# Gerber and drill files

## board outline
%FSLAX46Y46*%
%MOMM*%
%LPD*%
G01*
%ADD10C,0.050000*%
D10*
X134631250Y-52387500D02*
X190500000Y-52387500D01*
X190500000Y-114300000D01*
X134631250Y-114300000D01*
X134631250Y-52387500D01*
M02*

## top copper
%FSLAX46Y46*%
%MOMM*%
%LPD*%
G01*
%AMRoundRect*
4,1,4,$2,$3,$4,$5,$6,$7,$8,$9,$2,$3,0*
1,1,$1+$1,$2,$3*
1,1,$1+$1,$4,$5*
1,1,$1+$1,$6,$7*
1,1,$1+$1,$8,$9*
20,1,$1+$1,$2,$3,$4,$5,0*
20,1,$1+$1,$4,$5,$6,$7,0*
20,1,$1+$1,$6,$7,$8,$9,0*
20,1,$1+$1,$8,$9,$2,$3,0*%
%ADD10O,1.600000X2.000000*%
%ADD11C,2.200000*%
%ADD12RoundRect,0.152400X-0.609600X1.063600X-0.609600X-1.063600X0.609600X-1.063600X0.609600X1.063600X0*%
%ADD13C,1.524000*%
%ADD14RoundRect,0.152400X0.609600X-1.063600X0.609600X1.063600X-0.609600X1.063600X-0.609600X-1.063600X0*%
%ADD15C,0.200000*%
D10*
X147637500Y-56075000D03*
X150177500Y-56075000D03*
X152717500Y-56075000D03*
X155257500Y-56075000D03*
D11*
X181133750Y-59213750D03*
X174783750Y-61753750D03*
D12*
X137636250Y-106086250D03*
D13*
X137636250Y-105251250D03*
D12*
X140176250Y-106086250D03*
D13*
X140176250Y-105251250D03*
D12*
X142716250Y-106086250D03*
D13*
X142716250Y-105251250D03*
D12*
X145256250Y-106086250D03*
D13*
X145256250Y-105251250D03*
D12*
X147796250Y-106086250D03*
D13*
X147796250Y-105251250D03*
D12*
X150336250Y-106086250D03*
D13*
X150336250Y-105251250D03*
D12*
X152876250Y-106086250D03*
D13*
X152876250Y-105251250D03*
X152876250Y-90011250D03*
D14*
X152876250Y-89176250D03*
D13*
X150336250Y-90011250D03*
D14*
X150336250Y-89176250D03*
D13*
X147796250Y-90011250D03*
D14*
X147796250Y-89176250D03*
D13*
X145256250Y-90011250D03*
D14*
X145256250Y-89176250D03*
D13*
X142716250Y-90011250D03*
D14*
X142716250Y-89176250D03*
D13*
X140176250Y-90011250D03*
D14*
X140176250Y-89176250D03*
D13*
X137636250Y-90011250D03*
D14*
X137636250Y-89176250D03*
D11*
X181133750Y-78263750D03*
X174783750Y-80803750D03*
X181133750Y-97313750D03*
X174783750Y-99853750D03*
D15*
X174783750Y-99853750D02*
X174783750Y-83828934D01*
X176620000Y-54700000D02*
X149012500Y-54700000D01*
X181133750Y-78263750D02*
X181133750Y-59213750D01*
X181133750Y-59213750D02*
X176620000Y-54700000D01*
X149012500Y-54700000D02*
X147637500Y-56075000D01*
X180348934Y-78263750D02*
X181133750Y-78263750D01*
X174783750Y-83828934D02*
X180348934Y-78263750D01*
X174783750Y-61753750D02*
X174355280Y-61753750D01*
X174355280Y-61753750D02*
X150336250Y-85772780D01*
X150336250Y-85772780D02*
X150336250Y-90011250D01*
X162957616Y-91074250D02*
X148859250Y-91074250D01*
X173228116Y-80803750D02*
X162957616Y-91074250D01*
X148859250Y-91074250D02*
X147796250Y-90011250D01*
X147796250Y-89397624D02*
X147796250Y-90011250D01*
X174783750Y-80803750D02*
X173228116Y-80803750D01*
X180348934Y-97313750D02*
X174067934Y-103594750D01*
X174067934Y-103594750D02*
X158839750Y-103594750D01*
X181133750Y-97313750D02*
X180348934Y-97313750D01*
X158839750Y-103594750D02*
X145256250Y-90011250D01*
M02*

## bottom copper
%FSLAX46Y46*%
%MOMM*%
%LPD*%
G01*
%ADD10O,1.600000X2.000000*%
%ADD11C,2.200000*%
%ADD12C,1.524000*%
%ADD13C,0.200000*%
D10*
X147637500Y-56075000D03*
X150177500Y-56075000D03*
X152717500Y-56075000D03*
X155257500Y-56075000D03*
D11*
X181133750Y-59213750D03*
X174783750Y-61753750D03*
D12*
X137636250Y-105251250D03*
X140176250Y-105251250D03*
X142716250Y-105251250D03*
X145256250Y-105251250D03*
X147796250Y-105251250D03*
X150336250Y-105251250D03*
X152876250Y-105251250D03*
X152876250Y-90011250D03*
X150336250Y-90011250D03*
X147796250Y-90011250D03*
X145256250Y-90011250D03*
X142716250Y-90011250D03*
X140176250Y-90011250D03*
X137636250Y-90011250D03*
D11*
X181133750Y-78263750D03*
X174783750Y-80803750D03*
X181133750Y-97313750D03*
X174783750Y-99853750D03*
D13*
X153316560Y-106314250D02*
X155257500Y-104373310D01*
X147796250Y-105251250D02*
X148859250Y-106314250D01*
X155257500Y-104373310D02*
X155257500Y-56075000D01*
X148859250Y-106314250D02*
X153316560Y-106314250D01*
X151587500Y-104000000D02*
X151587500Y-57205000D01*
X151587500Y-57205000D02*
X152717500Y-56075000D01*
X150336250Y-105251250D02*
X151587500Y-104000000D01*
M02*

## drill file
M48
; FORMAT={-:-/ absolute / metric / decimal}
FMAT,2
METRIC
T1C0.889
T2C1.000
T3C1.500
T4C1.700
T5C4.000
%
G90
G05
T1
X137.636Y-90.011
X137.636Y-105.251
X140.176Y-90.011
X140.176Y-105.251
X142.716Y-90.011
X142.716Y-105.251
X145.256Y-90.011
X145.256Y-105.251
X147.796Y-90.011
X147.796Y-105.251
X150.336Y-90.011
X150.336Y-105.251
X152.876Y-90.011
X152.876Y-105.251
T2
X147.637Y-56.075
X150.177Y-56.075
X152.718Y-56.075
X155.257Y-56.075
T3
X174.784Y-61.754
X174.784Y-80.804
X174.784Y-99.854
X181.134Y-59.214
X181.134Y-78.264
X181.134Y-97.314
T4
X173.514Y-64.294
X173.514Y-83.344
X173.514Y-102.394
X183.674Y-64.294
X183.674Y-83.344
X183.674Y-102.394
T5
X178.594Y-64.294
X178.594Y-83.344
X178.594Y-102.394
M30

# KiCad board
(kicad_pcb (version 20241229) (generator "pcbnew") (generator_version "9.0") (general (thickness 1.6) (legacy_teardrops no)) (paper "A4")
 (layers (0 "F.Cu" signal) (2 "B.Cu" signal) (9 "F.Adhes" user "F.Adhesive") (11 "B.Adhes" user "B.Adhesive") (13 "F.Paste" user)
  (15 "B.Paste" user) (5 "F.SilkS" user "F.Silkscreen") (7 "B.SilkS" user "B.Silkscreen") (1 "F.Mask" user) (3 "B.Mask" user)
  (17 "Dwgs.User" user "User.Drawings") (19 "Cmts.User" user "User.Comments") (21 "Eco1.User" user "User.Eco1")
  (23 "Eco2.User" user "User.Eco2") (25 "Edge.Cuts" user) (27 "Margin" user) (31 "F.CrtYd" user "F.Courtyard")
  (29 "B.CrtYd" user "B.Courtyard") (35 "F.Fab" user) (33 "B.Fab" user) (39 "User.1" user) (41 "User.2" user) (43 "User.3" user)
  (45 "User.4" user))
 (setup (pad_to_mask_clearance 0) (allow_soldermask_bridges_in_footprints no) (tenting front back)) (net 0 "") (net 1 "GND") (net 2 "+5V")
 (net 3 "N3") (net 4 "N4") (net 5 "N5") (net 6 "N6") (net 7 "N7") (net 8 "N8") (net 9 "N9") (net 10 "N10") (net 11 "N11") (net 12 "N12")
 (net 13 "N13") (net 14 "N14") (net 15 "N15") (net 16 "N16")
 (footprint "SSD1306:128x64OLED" (layer "F.Cu") (at 151.2575 66.675)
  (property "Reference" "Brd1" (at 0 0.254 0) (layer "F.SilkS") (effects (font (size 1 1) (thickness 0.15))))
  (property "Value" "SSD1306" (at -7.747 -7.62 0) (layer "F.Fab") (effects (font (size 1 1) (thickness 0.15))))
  (pad "1" thru_hole oval (at -3.62 -10.6 90) (size 2 1.6) (drill 1) (layers "*.Cu" "*.Mask") (remove_unused_layers no) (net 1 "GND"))
  (pad "2" thru_hole oval (at -1.08 -10.6 90) (size 2 1.6) (drill 1) (layers "*.Cu" "*.Mask") (remove_unused_layers no) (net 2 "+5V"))
  (pad "3" thru_hole oval (at 1.46 -10.6 90) (size 2 1.6) (drill 1) (layers "*.Cu" "*.Mask") (remove_unused_layers no) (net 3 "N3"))
  (pad "4" thru_hole oval (at 4 -10.6 90) (size 2 1.6) (drill 1) (layers "*.Cu" "*.Mask") (remove_unused_layers no) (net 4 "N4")))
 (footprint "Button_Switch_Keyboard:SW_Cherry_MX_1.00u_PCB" (layer "F.Cu") (at 181.13375 59.21375)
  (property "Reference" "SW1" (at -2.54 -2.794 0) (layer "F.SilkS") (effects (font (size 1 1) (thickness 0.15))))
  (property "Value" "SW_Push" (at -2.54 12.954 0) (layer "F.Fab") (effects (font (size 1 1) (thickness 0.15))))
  (pad "" np_thru_hole circle (at -7.62 5.08) (size 1.7 1.7) (drill 1.7) (layers "*.Cu" "*.Mask"))
  (pad "" np_thru_hole circle (at -2.54 5.08) (size 4 4) (drill 4) (layers "*.Cu" "*.Mask"))
  (pad "" np_thru_hole circle (at 2.54 5.08) (size 1.7 1.7) (drill 1.7) (layers "*.Cu" "*.Mask"))
  (pad "1" thru_hole circle (at 0 0) (size 2.2 2.2) (drill 1.5) (layers "*.Cu" "*.Mask") (remove_unused_layers no) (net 1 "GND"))
  (pad "2" thru_hole circle (at -6.35 2.54) (size 2.2 2.2) (drill 1.5) (layers "*.Cu" "*.Mask") (remove_unused_layers no) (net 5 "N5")))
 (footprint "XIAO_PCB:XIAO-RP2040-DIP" (layer "F.Cu") (at 145.25625 97.63125 90)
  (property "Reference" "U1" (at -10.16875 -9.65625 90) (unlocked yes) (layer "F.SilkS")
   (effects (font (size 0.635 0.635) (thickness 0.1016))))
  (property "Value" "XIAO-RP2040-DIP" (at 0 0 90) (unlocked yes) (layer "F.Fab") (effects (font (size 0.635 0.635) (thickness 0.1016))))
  (pad "1" smd roundrect (at -8.455 -7.62 270) (size 2.432 1.524) (layers "F.Cu" "F.Mask") (roundrect_rratio 0.1) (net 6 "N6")
   (thermal_bridge_angle 45))
  (pad "1" thru_hole circle (at -7.62 -7.62 270) (size 1.524 1.524) (drill 0.889) (layers "*.Cu" "*.Mask") (remove_unused_layers no)
   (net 6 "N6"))
  (pad "2" smd roundrect (at -8.455 -5.08 270) (size 2.432 1.524) (layers "F.Cu" "F.Mask") (roundrect_rratio 0.1) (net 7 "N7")
   (thermal_bridge_angle 45))
  (pad "2" thru_hole circle (at -7.62 -5.08 270) (size 1.524 1.524) (drill 0.889) (layers "*.Cu" "*.Mask") (remove_unused_layers no)
   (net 7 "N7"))
  (pad "3" smd roundrect (at -8.455 -2.54 270) (size 2.432 1.524) (layers "F.Cu" "F.Mask") (roundrect_rratio 0.1) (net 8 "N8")
   (thermal_bridge_angle 45))
  (pad "3" thru_hole circle (at -7.62 -2.54 270) (size 1.524 1.524) (drill 0.889) (layers "*.Cu" "*.Mask") (remove_unused_layers no)
   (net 8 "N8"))
  (pad "4" smd roundrect (at -8.455 0 270) (size 2.432 1.524) (layers "F.Cu" "F.Mask") (roundrect_rratio 0.1) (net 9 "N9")
   (thermal_bridge_angle 45))
  (pad "4" thru_hole circle (at -7.62 0 270) (size 1.524 1.524) (drill 0.889) (layers "*.Cu" "*.Mask") (remove_unused_layers no)
   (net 9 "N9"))
  (pad "5" smd roundrect (at -8.455 2.54 270) (size 2.432 1.524) (layers "F.Cu" "F.Mask") (roundrect_rratio 0.1) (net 4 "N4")
   (thermal_bridge_angle 45))
  (pad "5" thru_hole circle (at -7.62 2.54 270) (size 1.524 1.524) (drill 0.889) (layers "*.Cu" "*.Mask") (remove_unused_layers no)
   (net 4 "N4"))
  (pad "6" smd roundrect (at -8.455 5.08 270) (size 2.432 1.524) (layers "F.Cu" "F.Mask") (roundrect_rratio 0.1) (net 3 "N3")
   (thermal_bridge_angle 45))
  (pad "6" thru_hole circle (at -7.62 5.08 270) (size 1.524 1.524) (drill 0.889) (layers "*.Cu" "*.Mask") (remove_unused_layers no)
   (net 3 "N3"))
  (pad "7" smd roundrect (at -8.455 7.62 270) (size 2.432 1.524) (layers "F.Cu" "F.Mask") (roundrect_rratio 0.1) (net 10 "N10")
   (thermal_bridge_angle 45))
  (pad "7" thru_hole circle (at -7.62 7.62 270) (size 1.524 1.524) (drill 0.889) (layers "*.Cu" "*.Mask") (remove_unused_layers no)
   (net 10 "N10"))
  (pad "8" thru_hole circle (at 7.62 7.62 90) (size 1.524 1.524) (drill 0.889) (layers "*.Cu" "*.Mask") (remove_unused_layers no)
   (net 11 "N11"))
  (pad "8" smd roundrect (at 8.455 7.62 90) (size 2.432 1.524) (layers "F.Cu" "F.Mask") (roundrect_rratio 0.1) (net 11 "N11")
   (thermal_bridge_angle 45))
  (pad "9" thru_hole circle (at 7.62 5.08 90) (size 1.524 1.524) (drill 0.889) (layers "*.Cu" "*.Mask") (remove_unused_layers no)
   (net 5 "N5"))
  (pad "9" smd roundrect (at 8.455 5.08 90) (size 2.432 1.524) (layers "F.Cu" "F.Mask") (roundrect_rratio 0.1) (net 5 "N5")
   (thermal_bridge_angle 45))
  (pad "10" thru_hole circle (at 7.62 2.54 90) (size 1.524 1.524) (drill 0.889) (layers "*.Cu" "*.Mask") (remove_unused_layers no)
   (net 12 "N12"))
  (pad "10" smd roundrect (at 8.455 2.54 90) (size 2.432 1.524) (layers "F.Cu" "F.Mask") (roundrect_rratio 0.1) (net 12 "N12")
   (thermal_bridge_angle 45))
  (pad "11" thru_hole circle (at 7.62 0 90) (size 1.524 1.524) (drill 0.889) (layers "*.Cu" "*.Mask") (remove_unused_layers no)
   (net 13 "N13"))
  (pad "11" smd roundrect (at 8.455 0 90) (size 2.432 1.524) (layers "F.Cu" "F.Mask") (roundrect_rratio 0.1) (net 13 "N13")
   (thermal_bridge_angle 45))
  (pad "12" thru_hole circle (at 7.62 -2.54 90) (size 1.524 1.524) (drill 0.889) (layers "*.Cu" "*.Mask") (remove_unused_layers no)
   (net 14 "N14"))
  (pad "12" smd roundrect (at 8.455 -2.54 90) (size 2.432 1.524) (layers "F.Cu" "F.Mask") (roundrect_rratio 0.1) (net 14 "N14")
   (thermal_bridge_angle 45))
  (pad "13" thru_hole circle (at 7.62 -5.08 90) (size 1.524 1.524) (drill 0.889) (layers "*.Cu" "*.Mask") (remove_unused_layers no)
   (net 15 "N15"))
  (pad "13" smd roundrect (at 8.455 -5.08 90) (size 2.432 1.524) (layers "F.Cu" "F.Mask") (roundrect_rratio 0.1) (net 15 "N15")
   (thermal_bridge_angle 45))
  (pad "14" thru_hole circle (at 7.62 -7.62 90) (size 1.524 1.524) (drill 0.889) (layers "*.Cu" "*.Mask") (remove_unused_layers no)
   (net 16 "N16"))
  (pad "14" smd roundrect (at 8.455 -7.62 90) (size 2.432 1.524) (layers "F.Cu" "F.Mask") (roundrect_rratio 0.1) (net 16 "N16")
   (thermal_bridge_angle 45)))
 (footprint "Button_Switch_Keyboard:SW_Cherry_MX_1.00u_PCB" (layer "F.Cu") (at 181.13375 78.26375)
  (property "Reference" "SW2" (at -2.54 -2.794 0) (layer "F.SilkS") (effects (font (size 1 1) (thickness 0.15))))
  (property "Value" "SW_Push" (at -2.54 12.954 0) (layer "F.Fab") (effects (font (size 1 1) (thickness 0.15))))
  (pad "" np_thru_hole circle (at -7.62 5.08) (size 1.7 1.7) (drill 1.7) (layers "*.Cu" "*.Mask"))
  (pad "" np_thru_hole circle (at -2.54 5.08) (size 4 4) (drill 4) (layers "*.Cu" "*.Mask"))
  (pad "" np_thru_hole circle (at 2.54 5.08) (size 1.7 1.7) (drill 1.7) (layers "*.Cu" "*.Mask"))
  (pad "1" thru_hole circle (at 0 0) (size 2.2 2.2) (drill 1.5) (layers "*.Cu" "*.Mask") (remove_unused_layers no) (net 1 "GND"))
  (pad "2" thru_hole circle (at -6.35 2.54) (size 2.2 2.2) (drill 1.5) (layers "*.Cu" "*.Mask") (remove_unused_layers no) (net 12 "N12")))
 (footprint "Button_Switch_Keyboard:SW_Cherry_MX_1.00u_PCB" (layer "F.Cu") (at 181.13375 97.31375)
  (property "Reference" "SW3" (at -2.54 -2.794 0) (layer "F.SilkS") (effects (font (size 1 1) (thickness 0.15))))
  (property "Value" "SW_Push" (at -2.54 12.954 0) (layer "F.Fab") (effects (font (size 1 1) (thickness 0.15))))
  (pad "" np_thru_hole circle (at -7.62 5.08) (size 1.7 1.7) (drill 1.7) (layers "*.Cu" "*.Mask"))
  (pad "" np_thru_hole circle (at -2.54 5.08) (size 4 4) (drill 4) (layers "*.Cu" "*.Mask"))
  (pad "" np_thru_hole circle (at 2.54 5.08) (size 1.7 1.7) (drill 1.7) (layers "*.Cu" "*.Mask"))
  (pad "1" thru_hole circle (at 0 0) (size 2.2 2.2) (drill 1.5) (layers "*.Cu" "*.Mask") (remove_unused_layers no) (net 13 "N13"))
  (pad "2" thru_hole circle (at -6.35 2.54) (size 2.2 2.2) (drill 1.5) (layers "*.Cu" "*.Mask") (remove_unused_layers no) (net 1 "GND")))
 (gr_rect (start 134.63125 52.3875) (end 190.5 114.3) (stroke (width 0.05) (type default)) (fill no) (layer "Edge.Cuts"))
 (segment (start 153.31656 106.31425) (end 155.2575 104.37331) (width 0.2) (layer "B.Cu") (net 4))
 (segment (start 147.79625 105.25125) (end 148.85925 106.31425) (width 0.2) (layer "B.Cu") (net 4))
 (segment (start 155.2575 104.37331) (end 155.2575 56.075) (width 0.2) (layer "B.Cu") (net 4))
 (segment (start 148.85925 106.31425) (end 153.31656 106.31425) (width 0.2) (layer "B.Cu") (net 4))
 (segment (start 174.78375 99.85375) (end 174.78375 83.828934) (width 0.2) (layer "F.Cu") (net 1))
 (segment (start 176.62 54.7) (end 149.0125 54.7) (width 0.2) (layer "F.Cu") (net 1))
 (segment (start 181.13375 78.26375) (end 181.13375 59.21375) (width 0.2) (layer "F.Cu") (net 1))
 (segment (start 181.13375 59.21375) (end 176.62 54.7) (width 0.2) (layer "F.Cu") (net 1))
 (segment (start 149.0125 54.7) (end 147.6375 56.075) (width 0.2) (layer "F.Cu") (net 1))
 (segment (start 180.348934 78.26375) (end 181.13375 78.26375) (width 0.2) (layer "F.Cu") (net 1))
 (segment (start 174.78375 83.828934) (end 180.348934 78.26375) (width 0.2) (layer "F.Cu") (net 1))
 (segment (start 151.5875 104) (end 151.5875 57.205) (width 0.2) (layer "B.Cu") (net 3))
 (segment (start 151.5875 57.205) (end 152.7175 56.075) (width 0.2) (layer "B.Cu") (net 3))
 (segment (start 150.33625 105.25125) (end 151.5875 104) (width 0.2) (layer "B.Cu") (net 3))
 (segment (start 174.78375 61.75375) (end 174.35528 61.75375) (width 0.2) (layer "F.Cu") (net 5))
 (segment (start 174.35528 61.75375) (end 150.33625 85.77278) (width 0.2) (layer "F.Cu") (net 5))
 (segment (start 150.33625 85.77278) (end 150.33625 90.01125) (width 0.2) (layer "F.Cu") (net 5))
 (segment (start 162.957616 91.07425) (end 148.85925 91.07425) (width 0.2) (layer "F.Cu") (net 12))
 (segment (start 173.228116 80.80375) (end 162.957616 91.07425) (width 0.2) (layer "F.Cu") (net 12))
 (segment (start 148.85925 91.07425) (end 147.79625 90.01125) (width 0.2) (layer "F.Cu") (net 12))
 (segment (start 147.79625 89.397624) (end 147.79625 90.01125) (width 0.2) (layer "F.Cu") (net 12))
 (segment (start 174.78375 80.80375) (end 173.228116 80.80375) (width 0.2) (layer "F.Cu") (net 12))
 (segment (start 180.348934 97.31375) (end 174.067934 103.59475) (width 0.2) (layer "F.Cu") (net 13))
 (segment (start 174.067934 103.59475) (end 158.83975 103.59475) (width 0.2) (layer "F.Cu") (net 13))
 (segment (start 181.13375 97.31375) (end 180.348934 97.31375) (width 0.2) (layer "F.Cu") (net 13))
 (segment (start 158.83975 103.59475) (end 145.25625 90.01125) (width 0.2) (layer "F.Cu") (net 13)))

